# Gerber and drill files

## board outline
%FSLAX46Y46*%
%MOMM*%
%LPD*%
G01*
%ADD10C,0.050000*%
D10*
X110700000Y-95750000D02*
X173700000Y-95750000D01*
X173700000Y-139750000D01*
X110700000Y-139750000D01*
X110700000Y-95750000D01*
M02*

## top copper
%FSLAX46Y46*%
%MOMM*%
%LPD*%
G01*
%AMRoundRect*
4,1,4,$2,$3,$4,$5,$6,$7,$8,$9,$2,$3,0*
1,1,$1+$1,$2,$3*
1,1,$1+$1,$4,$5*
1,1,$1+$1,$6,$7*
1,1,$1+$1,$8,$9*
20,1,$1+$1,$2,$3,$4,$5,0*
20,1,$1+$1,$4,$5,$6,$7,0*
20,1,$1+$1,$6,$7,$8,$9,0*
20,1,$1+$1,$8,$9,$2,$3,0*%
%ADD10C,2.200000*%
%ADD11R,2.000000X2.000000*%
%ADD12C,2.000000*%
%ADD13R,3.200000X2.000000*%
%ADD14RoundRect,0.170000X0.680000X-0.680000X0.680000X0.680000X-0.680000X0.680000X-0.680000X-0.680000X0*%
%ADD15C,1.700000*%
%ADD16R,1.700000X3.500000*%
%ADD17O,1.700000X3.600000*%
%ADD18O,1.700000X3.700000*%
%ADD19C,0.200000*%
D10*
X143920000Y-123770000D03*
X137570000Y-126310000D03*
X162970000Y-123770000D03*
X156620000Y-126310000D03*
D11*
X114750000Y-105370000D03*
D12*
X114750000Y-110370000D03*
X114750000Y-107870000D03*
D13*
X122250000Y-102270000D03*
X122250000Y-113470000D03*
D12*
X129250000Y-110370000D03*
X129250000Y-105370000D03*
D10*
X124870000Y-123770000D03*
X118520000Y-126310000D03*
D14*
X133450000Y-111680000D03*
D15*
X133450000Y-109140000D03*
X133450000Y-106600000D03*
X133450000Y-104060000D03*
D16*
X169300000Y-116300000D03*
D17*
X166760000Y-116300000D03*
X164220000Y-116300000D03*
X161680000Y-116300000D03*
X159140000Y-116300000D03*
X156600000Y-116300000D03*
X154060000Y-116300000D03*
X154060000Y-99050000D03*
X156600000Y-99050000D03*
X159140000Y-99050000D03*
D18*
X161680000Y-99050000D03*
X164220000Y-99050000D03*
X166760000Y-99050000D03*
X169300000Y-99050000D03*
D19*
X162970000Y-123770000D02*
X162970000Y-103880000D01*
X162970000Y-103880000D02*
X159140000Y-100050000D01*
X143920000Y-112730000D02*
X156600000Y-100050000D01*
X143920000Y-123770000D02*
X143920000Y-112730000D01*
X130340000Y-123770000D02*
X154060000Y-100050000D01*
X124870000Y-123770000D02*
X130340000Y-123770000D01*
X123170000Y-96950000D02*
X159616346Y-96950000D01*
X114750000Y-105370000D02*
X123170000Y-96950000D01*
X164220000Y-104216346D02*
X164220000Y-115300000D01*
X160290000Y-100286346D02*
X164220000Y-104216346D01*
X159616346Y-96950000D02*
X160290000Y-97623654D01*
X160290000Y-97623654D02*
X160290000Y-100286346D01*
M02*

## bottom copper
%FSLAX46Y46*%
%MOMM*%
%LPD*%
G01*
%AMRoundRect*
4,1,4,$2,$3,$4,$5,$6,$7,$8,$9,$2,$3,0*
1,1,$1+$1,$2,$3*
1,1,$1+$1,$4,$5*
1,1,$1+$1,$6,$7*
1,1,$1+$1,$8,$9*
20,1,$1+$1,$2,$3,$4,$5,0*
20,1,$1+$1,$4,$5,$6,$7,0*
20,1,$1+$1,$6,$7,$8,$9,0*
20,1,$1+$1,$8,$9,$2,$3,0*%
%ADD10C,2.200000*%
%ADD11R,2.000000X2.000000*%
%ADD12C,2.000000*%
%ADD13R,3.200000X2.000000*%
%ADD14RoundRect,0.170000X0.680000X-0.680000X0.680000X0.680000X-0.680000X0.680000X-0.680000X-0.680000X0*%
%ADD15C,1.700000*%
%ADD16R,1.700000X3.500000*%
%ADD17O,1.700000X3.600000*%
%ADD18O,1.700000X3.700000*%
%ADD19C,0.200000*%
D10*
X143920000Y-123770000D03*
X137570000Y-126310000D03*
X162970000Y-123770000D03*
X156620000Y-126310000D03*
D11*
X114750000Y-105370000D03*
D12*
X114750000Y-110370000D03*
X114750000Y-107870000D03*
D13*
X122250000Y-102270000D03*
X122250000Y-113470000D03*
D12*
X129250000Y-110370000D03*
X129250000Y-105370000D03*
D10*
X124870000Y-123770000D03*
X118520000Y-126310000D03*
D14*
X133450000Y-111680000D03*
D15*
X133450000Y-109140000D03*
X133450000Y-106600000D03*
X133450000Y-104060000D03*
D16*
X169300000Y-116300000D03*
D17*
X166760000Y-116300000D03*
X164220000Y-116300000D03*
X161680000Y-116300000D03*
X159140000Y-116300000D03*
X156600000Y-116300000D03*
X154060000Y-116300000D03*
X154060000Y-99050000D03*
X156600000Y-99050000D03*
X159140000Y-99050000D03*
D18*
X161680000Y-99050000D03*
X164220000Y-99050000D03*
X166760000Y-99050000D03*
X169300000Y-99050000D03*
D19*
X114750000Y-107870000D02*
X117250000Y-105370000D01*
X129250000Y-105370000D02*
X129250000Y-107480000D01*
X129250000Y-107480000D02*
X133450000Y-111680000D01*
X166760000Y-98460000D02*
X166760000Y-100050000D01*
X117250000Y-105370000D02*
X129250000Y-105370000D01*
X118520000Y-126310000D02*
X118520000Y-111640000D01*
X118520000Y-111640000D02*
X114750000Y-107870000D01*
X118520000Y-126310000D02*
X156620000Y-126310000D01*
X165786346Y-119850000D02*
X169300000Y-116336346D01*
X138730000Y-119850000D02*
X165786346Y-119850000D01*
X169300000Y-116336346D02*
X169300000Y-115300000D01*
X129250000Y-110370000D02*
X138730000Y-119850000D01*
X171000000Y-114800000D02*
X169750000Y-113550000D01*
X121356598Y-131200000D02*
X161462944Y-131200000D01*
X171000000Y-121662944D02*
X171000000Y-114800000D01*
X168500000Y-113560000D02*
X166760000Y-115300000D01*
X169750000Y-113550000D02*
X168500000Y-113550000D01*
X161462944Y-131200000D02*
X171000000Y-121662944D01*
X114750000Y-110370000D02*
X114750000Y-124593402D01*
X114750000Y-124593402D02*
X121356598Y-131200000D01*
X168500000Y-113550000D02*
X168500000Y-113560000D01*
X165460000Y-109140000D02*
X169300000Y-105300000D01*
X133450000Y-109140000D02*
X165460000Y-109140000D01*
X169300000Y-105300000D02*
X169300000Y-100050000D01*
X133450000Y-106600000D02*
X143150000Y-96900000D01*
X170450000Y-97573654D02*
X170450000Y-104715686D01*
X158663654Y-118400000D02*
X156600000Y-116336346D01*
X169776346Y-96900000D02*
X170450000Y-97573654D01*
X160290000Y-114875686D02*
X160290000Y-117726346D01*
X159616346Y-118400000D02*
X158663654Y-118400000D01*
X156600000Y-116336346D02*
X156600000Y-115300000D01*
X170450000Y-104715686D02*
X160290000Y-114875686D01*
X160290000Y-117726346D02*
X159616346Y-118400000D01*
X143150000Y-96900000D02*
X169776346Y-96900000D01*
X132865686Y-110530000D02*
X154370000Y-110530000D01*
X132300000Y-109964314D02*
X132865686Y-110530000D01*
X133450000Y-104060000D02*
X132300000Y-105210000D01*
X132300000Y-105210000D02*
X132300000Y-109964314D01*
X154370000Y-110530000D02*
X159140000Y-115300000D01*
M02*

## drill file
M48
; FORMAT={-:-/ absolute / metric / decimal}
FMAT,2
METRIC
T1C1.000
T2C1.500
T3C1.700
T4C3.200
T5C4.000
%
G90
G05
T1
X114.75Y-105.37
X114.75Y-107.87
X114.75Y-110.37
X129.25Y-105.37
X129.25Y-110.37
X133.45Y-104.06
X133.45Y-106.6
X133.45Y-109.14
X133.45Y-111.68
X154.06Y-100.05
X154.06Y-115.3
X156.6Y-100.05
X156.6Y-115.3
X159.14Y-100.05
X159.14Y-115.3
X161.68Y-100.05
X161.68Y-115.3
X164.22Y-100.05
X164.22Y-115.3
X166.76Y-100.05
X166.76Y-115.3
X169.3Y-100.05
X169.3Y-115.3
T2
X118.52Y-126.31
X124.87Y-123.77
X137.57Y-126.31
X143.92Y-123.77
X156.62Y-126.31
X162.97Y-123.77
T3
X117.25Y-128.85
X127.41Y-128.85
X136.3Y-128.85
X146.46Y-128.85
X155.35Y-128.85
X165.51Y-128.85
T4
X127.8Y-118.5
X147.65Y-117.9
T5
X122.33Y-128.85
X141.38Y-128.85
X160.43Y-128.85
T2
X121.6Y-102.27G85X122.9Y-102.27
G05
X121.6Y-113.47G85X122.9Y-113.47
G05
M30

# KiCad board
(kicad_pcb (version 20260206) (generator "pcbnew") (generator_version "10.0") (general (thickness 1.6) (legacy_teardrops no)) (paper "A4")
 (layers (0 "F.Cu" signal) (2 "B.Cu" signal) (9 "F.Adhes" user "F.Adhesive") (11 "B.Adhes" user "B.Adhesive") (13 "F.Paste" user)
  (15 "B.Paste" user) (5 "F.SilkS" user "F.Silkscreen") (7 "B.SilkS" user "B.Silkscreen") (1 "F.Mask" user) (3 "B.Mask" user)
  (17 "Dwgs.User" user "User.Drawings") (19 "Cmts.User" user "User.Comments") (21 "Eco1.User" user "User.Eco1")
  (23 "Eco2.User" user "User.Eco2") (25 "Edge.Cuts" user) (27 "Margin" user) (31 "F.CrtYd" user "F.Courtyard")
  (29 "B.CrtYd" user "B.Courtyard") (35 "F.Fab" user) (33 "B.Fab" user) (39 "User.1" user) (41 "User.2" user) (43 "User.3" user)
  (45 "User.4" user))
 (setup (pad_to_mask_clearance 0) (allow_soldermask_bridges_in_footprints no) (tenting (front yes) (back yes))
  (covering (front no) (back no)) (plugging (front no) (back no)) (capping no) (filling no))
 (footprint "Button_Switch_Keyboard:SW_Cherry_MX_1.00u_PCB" (layer "F.Cu") (at 143.92 123.77)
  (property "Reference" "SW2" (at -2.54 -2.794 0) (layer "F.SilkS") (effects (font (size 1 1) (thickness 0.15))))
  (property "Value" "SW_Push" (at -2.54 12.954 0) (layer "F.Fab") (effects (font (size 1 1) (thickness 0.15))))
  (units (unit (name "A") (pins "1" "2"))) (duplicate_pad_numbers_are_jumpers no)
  (pad "" np_thru_hole circle (at -7.62 5.08) (size 1.7 1.7) (drill 1.7) (layers "*.Cu" "*.Mask"))
  (pad "" np_thru_hole circle (at -2.54 5.08) (size 4 4) (drill 4) (layers "*.Cu" "*.Mask"))
  (pad "" np_thru_hole circle (at 2.54 5.08) (size 1.7 1.7) (drill 1.7) (layers "*.Cu" "*.Mask"))
  (pad "1" thru_hole circle (at 0 0) (size 2.2 2.2) (drill 1.5) (layers "*.Cu" "*.Mask") (remove_unused_layers no)
   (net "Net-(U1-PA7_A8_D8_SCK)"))
  (pad "2" thru_hole circle (at -6.35 2.54) (size 2.2 2.2) (drill 1.5) (layers "*.Cu" "*.Mask") (remove_unused_layers no) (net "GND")))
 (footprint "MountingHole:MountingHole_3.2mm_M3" (layer "F.Cu") (at 147.65 117.9)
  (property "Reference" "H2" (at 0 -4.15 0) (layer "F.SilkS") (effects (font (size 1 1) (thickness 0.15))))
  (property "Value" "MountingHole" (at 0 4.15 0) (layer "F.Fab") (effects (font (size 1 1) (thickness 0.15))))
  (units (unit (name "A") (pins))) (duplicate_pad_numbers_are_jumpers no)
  (pad "" np_thru_hole circle (at 0 0) (size 3.2 3.2) (drill 3.2) (layers "*.Cu" "*.Mask")))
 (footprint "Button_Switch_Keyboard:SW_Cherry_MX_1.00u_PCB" (layer "F.Cu") (at 162.97 123.77)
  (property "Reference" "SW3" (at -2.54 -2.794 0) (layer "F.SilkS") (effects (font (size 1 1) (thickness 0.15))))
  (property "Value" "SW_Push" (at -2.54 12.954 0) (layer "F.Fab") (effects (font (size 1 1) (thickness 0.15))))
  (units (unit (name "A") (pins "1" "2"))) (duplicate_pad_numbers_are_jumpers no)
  (pad "" np_thru_hole circle (at -7.62 5.08) (size 1.7 1.7) (drill 1.7) (layers "*.Cu" "*.Mask"))
  (pad "" np_thru_hole circle (at -2.54 5.08) (size 4 4) (drill 4) (layers "*.Cu" "*.Mask"))
  (pad "" np_thru_hole circle (at 2.54 5.08) (size 1.7 1.7) (drill 1.7) (layers "*.Cu" "*.Mask"))
  (pad "1" thru_hole circle (at 0 0) (size 2.2 2.2) (drill 1.5) (layers "*.Cu" "*.Mask") (remove_unused_layers no)
   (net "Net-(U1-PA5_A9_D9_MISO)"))
  (pad "2" thru_hole circle (at -6.35 2.54) (size 2.2 2.2) (drill 1.5) (layers "*.Cu" "*.Mask") (remove_unused_layers no) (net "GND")))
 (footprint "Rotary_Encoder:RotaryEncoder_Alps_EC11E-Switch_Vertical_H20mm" (layer "F.Cu") (at 114.75 105.37)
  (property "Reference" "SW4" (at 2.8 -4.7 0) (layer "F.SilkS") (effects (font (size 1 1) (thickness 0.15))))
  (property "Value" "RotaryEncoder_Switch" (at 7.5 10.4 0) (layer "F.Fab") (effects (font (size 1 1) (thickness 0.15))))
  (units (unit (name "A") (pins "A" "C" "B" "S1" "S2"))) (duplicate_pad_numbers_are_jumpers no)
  (pad "A" thru_hole rect (at 0 0) (size 2 2) (drill 1) (layers "*.Cu" "*.Mask") (remove_unused_layers no) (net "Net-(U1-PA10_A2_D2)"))
  (pad "B" thru_hole circle (at 0 5) (size 2 2) (drill 1) (layers "*.Cu" "*.Mask") (remove_unused_layers no) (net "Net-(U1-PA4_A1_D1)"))
  (pad "C" thru_hole circle (at 0 2.5) (size 2 2) (drill 1) (layers "*.Cu" "*.Mask") (remove_unused_layers no) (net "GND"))
  (pad "MP" thru_hole rect (at 7.5 -3.1) (size 3.2 2) (drill oval 2.8 1.5) (layers "*.Cu" "*.Mask") (remove_unused_layers no))
  (pad "MP" thru_hole rect (at 7.5 8.1) (size 3.2 2) (drill oval 2.8 1.5) (layers "*.Cu" "*.Mask") (remove_unused_layers no))
  (pad "S1" thru_hole circle (at 14.5 5) (size 2 2) (drill 1) (layers "*.Cu" "*.Mask") (remove_unused_layers no) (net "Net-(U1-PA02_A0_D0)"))
  (pad "S2" thru_hole circle (at 14.5 0) (size 2 2) (drill 1) (layers "*.Cu" "*.Mask") (remove_unused_layers no) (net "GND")))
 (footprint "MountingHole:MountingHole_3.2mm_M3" (layer "F.Cu") (at 127.8 118.5)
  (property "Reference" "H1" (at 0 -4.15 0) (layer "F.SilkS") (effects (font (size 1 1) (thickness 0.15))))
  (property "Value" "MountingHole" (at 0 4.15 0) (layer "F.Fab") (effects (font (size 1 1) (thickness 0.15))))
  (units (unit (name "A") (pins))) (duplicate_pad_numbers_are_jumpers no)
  (pad "" np_thru_hole circle (at 0 0) (size 3.2 3.2) (drill 3.2) (layers "*.Cu" "*.Mask")))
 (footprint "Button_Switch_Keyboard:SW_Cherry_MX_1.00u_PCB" (layer "F.Cu") (at 124.87 123.77)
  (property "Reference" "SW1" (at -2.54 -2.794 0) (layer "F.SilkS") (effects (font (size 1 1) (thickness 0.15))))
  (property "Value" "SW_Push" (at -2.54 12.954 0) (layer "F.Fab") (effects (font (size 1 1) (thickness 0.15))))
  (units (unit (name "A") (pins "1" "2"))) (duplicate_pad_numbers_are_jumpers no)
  (pad "" np_thru_hole circle (at -7.62 5.08) (size 1.7 1.7) (drill 1.7) (layers "*.Cu" "*.Mask"))
  (pad "" np_thru_hole circle (at -2.54 5.08) (size 4 4) (drill 4) (layers "*.Cu" "*.Mask"))
  (pad "" np_thru_hole circle (at 2.54 5.08) (size 1.7 1.7) (drill 1.7) (layers "*.Cu" "*.Mask"))
  (pad "1" thru_hole circle (at 0 0) (size 2.2 2.2) (drill 1.5) (layers "*.Cu" "*.Mask") (remove_unused_layers no)
   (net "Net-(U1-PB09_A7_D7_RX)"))
  (pad "2" thru_hole circle (at -6.35 2.54) (size 2.2 2.2) (drill 1.5) (layers "*.Cu" "*.Mask") (remove_unused_layers no) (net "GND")))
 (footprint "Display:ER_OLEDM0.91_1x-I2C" (layer "F.Cu") (at 133.45 111.68 90)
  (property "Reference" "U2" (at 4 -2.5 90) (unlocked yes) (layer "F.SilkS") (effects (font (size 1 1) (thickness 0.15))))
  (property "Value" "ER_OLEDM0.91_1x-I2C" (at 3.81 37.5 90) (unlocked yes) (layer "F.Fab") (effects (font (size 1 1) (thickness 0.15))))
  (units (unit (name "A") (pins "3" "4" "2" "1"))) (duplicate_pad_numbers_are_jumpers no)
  (pad "1" thru_hole roundrect (at 0 0 90) (size 1.7 1.7) (drill 1) (layers "*.Cu" "*.Mask") (remove_unused_layers no)
   (roundrect_rratio 0.1) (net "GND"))
  (pad "2" thru_hole circle (at 2.54 0 90) (size 1.7 1.7) (drill 1) (layers "*.Cu" "*.Mask") (remove_unused_layers no) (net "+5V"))
  (pad "3" thru_hole circle (at 5.08 0 90) (size 1.7 1.7) (drill 1) (layers "*.Cu" "*.Mask") (remove_unused_layers no)
   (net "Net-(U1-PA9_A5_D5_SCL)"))
  (pad "4" thru_hole circle (at 7.62 0 90) (size 1.7 1.7) (drill 1) (layers "*.Cu" "*.Mask") (remove_unused_layers no)
   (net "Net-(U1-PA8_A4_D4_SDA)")))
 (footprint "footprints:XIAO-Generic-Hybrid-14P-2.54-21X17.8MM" (layer "B.Cu") (at 161.68 107.675 90)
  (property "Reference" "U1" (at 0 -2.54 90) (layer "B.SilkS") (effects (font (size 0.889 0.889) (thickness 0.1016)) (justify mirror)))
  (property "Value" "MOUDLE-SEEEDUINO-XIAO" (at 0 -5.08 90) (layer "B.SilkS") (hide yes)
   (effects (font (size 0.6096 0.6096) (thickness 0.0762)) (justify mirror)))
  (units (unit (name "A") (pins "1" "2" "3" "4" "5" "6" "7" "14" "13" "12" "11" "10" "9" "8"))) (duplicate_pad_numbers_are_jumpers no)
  (pad "1" thru_hole rect (at -7.625 7.62 90) (size 3.5 1.7) (drill 1 (offset -1 0)) (layers "*.Cu" "*.Mask") (remove_unused_layers no)
   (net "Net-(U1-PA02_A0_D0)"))
  (pad "2" thru_hole oval (at -7.625 5.08 90) (size 3.6 1.7) (drill 1 (offset -1 0)) (layers "*.Cu" "*.Mask") (remove_unused_layers no)
   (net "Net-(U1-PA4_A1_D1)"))
  (pad "3" thru_hole oval (at -7.625 2.54 90) (size 3.6 1.7) (drill 1 (offset -1 0)) (layers "*.Cu" "*.Mask") (remove_unused_layers no)
   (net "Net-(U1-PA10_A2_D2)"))
  (pad "4" thru_hole oval (at -7.625 0 90) (size 3.6 1.7) (drill 1 (offset -1 0)) (layers "*.Cu" "*.Mask") (remove_unused_layers no)
   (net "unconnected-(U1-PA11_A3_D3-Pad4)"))
  (pad "5" thru_hole oval (at -7.625 -2.54 90) (size 3.6 1.7) (drill 1 (offset -1 0)) (layers "*.Cu" "*.Mask") (remove_unused_layers no)
   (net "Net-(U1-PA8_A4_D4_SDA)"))
  (pad "6" thru_hole oval (at -7.625 -5.08 270) (size 3.6 1.7) (drill 1 (offset 1 0)) (layers "*.Cu" "*.Mask") (remove_unused_layers no)
   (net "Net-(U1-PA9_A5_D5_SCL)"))
  (pad "7" thru_hole oval (at -7.625 -7.62 90) (size 3.6 1.7) (drill 1 (offset -1 0)) (layers "*.Cu" "*.Mask") (remove_unused_layers no)
   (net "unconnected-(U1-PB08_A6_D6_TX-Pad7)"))
  (pad "8" thru_hole oval (at 7.625 -7.62 90) (size 3.6 1.7) (drill 1 (offset 1 0)) (layers "*.Cu" "*.Mask") (remove_unused_layers no)
   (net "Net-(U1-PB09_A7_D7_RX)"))
  (pad "9" thru_hole oval (at 7.625 -5.08 90) (size 3.6 1.7) (drill 1 (offset 1 0)) (layers "*.Cu" "*.Mask") (remove_unused_layers no)
   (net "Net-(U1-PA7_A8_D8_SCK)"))
  (pad "10" thru_hole oval (at 7.625 -2.54 90) (size 3.6 1.7) (drill 1 (offset 1 0)) (layers "*.Cu" "*.Mask") (remove_unused_layers no)
   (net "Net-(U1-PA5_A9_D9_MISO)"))
  (pad "11" thru_hole oval (at 7.625 0 90) (size 3.7 1.7) (drill 1 (offset 1 0)) (layers "*.Cu" "*.Mask") (remove_unused_layers no)
   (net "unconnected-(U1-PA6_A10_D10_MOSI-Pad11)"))
  (pad "12" thru_hole oval (at 7.625 2.54 90) (size 3.7 1.7) (drill 1 (offset 1 0)) (layers "*.Cu" "*.Mask") (remove_unused_layers no)
   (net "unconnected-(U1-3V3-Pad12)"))
  (pad "13" thru_hole oval (at 7.625 5.08 90) (size 3.7 1.7) (drill 1 (offset 1 0)) (layers "*.Cu" "*.Mask") (remove_unused_layers no)
   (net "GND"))
  (pad "14" thru_hole oval (at 7.625 7.62 90) (size 3.7 1.7) (drill 1 (offset 1 0)) (layers "*.Cu" "*.Mask") (remove_unused_layers no)
   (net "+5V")))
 (gr_rect (start 110.7 95.75) (end 173.7 139.75) (stroke (width 0.05) (type solid)) (fill no) (layer "Edge.Cuts"))
 (segment (start 162.97 123.77) (end 162.97 103.88) (width 0.2) (layer "F.Cu") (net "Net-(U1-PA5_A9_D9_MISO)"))
 (segment (start 162.97 103.88) (end 159.14 100.05) (width 0.2) (layer "F.Cu") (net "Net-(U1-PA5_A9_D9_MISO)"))
 (segment (start 114.75 107.87) (end 117.25 105.37) (width 0.2) (layer "B.Cu") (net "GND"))
 (segment (start 129.25 105.37) (end 129.25 107.48) (width 0.2) (layer "B.Cu") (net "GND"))
 (segment (start 129.25 107.48) (end 133.45 111.68) (width 0.2) (layer "B.Cu") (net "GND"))
 (segment (start 166.76 98.46) (end 166.76 100.05) (width 0.2) (layer "B.Cu") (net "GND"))
 (segment (start 117.25 105.37) (end 129.25 105.37) (width 0.2) (layer "B.Cu") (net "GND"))
 (segment (start 118.52 126.31) (end 118.52 111.64) (width 0.2) (layer "B.Cu") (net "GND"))
 (segment (start 118.52 111.64) (end 114.75 107.87) (width 0.2) (layer "B.Cu") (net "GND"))
 (segment (start 118.52 126.31) (end 156.62 126.31) (width 0.2) (layer "B.Cu") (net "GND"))
 (segment (start 143.92 112.73) (end 156.6 100.05) (width 0.2) (layer "F.Cu") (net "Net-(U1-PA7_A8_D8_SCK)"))
 (segment (start 143.92 123.77) (end 143.92 112.73) (width 0.2) (layer "F.Cu") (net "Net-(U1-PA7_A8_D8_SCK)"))
 (segment (start 130.34 123.77) (end 154.06 100.05) (width 0.2) (layer "F.Cu") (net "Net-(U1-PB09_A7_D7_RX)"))
 (segment (start 124.87 123.77) (end 130.34 123.77) (width 0.2) (layer "F.Cu") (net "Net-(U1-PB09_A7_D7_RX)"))
 (segment (start 123.17 96.95) (end 159.616346 96.95) (width 0.2) (layer "F.Cu") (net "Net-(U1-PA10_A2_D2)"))
 (segment (start 114.75 105.37) (end 123.17 96.95) (width 0.2) (layer "F.Cu") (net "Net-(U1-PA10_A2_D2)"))
 (segment (start 164.22 104.216346) (end 164.22 115.3) (width 0.2) (layer "F.Cu") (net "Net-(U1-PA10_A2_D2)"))
 (segment (start 160.29 100.286346) (end 164.22 104.216346) (width 0.2) (layer "F.Cu") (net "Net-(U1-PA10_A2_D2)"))
 (segment (start 159.616346 96.95) (end 160.29 97.623654) (width 0.2) (layer "F.Cu") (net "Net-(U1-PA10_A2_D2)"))
 (segment (start 160.29 97.623654) (end 160.29 100.286346) (width 0.2) (layer "F.Cu") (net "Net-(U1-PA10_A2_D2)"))
 (segment (start 165.786346 119.85) (end 169.3 116.336346) (width 0.2) (layer "B.Cu") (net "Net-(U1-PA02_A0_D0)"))
 (segment (start 138.73 119.85) (end 165.786346 119.85) (width 0.2) (layer "B.Cu") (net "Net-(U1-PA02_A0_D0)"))
 (segment (start 169.3 116.336346) (end 169.3 115.3) (width 0.2) (layer "B.Cu") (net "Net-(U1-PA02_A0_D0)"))
 (segment (start 129.25 110.37) (end 138.73 119.85) (width 0.2) (layer "B.Cu") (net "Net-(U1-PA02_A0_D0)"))
 (segment (start 171 114.8) (end 169.75 113.55) (width 0.2) (layer "B.Cu") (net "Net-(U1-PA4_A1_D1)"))
 (segment (start 121.356598 131.2) (end 161.462944 131.2) (width 0.2) (layer "B.Cu") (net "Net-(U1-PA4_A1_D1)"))
 (segment (start 171 121.662944) (end 171 114.8) (width 0.2) (layer "B.Cu") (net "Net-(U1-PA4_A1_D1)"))
 (segment (start 168.5 113.56) (end 166.76 115.3) (width 0.2) (layer "B.Cu") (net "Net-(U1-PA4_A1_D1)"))
 (segment (start 169.75 113.55) (end 168.5 113.55) (width 0.2) (layer "B.Cu") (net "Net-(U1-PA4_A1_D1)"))
 (segment (start 161.462944 131.2) (end 171 121.662944) (width 0.2) (layer "B.Cu") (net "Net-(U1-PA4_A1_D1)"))
 (segment (start 114.75 110.37) (end 114.75 124.593402) (width 0.2) (layer "B.Cu") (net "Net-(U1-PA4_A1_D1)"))
 (segment (start 114.75 124.593402) (end 121.356598 131.2) (width 0.2) (layer "B.Cu") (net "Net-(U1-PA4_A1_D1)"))
 (segment (start 168.5 113.55) (end 168.5 113.56) (width 0.2) (layer "B.Cu") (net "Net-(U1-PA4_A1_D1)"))
 (segment (start 165.46 109.14) (end 169.3 105.3) (width 0.2) (layer "B.Cu") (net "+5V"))
 (segment (start 133.45 109.14) (end 165.46 109.14) (width 0.2) (layer "B.Cu") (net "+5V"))
 (segment (start 169.3 105.3) (end 169.3 100.05) (width 0.2) (layer "B.Cu") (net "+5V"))
 (segment (start 133.45 106.6) (end 143.15 96.9) (width 0.2) (layer "B.Cu") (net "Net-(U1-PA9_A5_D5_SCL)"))
 (segment (start 170.45 97.573654) (end 170.45 104.715686) (width 0.2) (layer "B.Cu") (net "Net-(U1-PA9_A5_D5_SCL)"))
 (segment (start 158.663654 118.4) (end 156.6 116.336346) (width 0.2) (layer "B.Cu") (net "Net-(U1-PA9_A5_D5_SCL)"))
 (segment (start 169.776346 96.9) (end 170.45 97.573654) (width 0.2) (layer "B.Cu") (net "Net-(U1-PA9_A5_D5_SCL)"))
 (segment (start 160.29 114.875686) (end 160.29 117.726346) (width 0.2) (layer "B.Cu") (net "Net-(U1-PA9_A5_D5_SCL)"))
 (segment (start 159.616346 118.4) (end 158.663654 118.4) (width 0.2) (layer "B.Cu") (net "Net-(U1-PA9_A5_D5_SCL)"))
 (segment (start 156.6 116.336346) (end 156.6 115.3) (width 0.2) (layer "B.Cu") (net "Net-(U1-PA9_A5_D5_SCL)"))
 (segment (start 170.45 104.715686) (end 160.29 114.875686) (width 0.2) (layer "B.Cu") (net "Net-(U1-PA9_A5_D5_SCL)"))
 (segment (start 160.29 117.726346) (end 159.616346 118.4) (width 0.2) (layer "B.Cu") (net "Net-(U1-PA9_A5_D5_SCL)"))
 (segment (start 143.15 96.9) (end 169.776346 96.9) (width 0.2) (layer "B.Cu") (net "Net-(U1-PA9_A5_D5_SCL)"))
 (segment (start 132.865686 110.53) (end 154.37 110.53) (width 0.2) (layer "B.Cu") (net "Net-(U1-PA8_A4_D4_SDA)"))
 (segment (start 132.3 109.964314) (end 132.865686 110.53) (width 0.2) (layer "B.Cu") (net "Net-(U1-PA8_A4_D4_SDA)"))
 (segment (start 133.45 104.06) (end 132.3 105.21) (width 0.2) (layer "B.Cu") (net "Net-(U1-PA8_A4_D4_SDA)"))
 (segment (start 132.3 105.21) (end 132.3 109.964314) (width 0.2) (layer "B.Cu") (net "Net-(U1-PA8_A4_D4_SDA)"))
 (segment (start 154.37 110.53) (end 159.14 115.3) (width 0.2) (layer "B.Cu") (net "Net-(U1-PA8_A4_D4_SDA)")))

